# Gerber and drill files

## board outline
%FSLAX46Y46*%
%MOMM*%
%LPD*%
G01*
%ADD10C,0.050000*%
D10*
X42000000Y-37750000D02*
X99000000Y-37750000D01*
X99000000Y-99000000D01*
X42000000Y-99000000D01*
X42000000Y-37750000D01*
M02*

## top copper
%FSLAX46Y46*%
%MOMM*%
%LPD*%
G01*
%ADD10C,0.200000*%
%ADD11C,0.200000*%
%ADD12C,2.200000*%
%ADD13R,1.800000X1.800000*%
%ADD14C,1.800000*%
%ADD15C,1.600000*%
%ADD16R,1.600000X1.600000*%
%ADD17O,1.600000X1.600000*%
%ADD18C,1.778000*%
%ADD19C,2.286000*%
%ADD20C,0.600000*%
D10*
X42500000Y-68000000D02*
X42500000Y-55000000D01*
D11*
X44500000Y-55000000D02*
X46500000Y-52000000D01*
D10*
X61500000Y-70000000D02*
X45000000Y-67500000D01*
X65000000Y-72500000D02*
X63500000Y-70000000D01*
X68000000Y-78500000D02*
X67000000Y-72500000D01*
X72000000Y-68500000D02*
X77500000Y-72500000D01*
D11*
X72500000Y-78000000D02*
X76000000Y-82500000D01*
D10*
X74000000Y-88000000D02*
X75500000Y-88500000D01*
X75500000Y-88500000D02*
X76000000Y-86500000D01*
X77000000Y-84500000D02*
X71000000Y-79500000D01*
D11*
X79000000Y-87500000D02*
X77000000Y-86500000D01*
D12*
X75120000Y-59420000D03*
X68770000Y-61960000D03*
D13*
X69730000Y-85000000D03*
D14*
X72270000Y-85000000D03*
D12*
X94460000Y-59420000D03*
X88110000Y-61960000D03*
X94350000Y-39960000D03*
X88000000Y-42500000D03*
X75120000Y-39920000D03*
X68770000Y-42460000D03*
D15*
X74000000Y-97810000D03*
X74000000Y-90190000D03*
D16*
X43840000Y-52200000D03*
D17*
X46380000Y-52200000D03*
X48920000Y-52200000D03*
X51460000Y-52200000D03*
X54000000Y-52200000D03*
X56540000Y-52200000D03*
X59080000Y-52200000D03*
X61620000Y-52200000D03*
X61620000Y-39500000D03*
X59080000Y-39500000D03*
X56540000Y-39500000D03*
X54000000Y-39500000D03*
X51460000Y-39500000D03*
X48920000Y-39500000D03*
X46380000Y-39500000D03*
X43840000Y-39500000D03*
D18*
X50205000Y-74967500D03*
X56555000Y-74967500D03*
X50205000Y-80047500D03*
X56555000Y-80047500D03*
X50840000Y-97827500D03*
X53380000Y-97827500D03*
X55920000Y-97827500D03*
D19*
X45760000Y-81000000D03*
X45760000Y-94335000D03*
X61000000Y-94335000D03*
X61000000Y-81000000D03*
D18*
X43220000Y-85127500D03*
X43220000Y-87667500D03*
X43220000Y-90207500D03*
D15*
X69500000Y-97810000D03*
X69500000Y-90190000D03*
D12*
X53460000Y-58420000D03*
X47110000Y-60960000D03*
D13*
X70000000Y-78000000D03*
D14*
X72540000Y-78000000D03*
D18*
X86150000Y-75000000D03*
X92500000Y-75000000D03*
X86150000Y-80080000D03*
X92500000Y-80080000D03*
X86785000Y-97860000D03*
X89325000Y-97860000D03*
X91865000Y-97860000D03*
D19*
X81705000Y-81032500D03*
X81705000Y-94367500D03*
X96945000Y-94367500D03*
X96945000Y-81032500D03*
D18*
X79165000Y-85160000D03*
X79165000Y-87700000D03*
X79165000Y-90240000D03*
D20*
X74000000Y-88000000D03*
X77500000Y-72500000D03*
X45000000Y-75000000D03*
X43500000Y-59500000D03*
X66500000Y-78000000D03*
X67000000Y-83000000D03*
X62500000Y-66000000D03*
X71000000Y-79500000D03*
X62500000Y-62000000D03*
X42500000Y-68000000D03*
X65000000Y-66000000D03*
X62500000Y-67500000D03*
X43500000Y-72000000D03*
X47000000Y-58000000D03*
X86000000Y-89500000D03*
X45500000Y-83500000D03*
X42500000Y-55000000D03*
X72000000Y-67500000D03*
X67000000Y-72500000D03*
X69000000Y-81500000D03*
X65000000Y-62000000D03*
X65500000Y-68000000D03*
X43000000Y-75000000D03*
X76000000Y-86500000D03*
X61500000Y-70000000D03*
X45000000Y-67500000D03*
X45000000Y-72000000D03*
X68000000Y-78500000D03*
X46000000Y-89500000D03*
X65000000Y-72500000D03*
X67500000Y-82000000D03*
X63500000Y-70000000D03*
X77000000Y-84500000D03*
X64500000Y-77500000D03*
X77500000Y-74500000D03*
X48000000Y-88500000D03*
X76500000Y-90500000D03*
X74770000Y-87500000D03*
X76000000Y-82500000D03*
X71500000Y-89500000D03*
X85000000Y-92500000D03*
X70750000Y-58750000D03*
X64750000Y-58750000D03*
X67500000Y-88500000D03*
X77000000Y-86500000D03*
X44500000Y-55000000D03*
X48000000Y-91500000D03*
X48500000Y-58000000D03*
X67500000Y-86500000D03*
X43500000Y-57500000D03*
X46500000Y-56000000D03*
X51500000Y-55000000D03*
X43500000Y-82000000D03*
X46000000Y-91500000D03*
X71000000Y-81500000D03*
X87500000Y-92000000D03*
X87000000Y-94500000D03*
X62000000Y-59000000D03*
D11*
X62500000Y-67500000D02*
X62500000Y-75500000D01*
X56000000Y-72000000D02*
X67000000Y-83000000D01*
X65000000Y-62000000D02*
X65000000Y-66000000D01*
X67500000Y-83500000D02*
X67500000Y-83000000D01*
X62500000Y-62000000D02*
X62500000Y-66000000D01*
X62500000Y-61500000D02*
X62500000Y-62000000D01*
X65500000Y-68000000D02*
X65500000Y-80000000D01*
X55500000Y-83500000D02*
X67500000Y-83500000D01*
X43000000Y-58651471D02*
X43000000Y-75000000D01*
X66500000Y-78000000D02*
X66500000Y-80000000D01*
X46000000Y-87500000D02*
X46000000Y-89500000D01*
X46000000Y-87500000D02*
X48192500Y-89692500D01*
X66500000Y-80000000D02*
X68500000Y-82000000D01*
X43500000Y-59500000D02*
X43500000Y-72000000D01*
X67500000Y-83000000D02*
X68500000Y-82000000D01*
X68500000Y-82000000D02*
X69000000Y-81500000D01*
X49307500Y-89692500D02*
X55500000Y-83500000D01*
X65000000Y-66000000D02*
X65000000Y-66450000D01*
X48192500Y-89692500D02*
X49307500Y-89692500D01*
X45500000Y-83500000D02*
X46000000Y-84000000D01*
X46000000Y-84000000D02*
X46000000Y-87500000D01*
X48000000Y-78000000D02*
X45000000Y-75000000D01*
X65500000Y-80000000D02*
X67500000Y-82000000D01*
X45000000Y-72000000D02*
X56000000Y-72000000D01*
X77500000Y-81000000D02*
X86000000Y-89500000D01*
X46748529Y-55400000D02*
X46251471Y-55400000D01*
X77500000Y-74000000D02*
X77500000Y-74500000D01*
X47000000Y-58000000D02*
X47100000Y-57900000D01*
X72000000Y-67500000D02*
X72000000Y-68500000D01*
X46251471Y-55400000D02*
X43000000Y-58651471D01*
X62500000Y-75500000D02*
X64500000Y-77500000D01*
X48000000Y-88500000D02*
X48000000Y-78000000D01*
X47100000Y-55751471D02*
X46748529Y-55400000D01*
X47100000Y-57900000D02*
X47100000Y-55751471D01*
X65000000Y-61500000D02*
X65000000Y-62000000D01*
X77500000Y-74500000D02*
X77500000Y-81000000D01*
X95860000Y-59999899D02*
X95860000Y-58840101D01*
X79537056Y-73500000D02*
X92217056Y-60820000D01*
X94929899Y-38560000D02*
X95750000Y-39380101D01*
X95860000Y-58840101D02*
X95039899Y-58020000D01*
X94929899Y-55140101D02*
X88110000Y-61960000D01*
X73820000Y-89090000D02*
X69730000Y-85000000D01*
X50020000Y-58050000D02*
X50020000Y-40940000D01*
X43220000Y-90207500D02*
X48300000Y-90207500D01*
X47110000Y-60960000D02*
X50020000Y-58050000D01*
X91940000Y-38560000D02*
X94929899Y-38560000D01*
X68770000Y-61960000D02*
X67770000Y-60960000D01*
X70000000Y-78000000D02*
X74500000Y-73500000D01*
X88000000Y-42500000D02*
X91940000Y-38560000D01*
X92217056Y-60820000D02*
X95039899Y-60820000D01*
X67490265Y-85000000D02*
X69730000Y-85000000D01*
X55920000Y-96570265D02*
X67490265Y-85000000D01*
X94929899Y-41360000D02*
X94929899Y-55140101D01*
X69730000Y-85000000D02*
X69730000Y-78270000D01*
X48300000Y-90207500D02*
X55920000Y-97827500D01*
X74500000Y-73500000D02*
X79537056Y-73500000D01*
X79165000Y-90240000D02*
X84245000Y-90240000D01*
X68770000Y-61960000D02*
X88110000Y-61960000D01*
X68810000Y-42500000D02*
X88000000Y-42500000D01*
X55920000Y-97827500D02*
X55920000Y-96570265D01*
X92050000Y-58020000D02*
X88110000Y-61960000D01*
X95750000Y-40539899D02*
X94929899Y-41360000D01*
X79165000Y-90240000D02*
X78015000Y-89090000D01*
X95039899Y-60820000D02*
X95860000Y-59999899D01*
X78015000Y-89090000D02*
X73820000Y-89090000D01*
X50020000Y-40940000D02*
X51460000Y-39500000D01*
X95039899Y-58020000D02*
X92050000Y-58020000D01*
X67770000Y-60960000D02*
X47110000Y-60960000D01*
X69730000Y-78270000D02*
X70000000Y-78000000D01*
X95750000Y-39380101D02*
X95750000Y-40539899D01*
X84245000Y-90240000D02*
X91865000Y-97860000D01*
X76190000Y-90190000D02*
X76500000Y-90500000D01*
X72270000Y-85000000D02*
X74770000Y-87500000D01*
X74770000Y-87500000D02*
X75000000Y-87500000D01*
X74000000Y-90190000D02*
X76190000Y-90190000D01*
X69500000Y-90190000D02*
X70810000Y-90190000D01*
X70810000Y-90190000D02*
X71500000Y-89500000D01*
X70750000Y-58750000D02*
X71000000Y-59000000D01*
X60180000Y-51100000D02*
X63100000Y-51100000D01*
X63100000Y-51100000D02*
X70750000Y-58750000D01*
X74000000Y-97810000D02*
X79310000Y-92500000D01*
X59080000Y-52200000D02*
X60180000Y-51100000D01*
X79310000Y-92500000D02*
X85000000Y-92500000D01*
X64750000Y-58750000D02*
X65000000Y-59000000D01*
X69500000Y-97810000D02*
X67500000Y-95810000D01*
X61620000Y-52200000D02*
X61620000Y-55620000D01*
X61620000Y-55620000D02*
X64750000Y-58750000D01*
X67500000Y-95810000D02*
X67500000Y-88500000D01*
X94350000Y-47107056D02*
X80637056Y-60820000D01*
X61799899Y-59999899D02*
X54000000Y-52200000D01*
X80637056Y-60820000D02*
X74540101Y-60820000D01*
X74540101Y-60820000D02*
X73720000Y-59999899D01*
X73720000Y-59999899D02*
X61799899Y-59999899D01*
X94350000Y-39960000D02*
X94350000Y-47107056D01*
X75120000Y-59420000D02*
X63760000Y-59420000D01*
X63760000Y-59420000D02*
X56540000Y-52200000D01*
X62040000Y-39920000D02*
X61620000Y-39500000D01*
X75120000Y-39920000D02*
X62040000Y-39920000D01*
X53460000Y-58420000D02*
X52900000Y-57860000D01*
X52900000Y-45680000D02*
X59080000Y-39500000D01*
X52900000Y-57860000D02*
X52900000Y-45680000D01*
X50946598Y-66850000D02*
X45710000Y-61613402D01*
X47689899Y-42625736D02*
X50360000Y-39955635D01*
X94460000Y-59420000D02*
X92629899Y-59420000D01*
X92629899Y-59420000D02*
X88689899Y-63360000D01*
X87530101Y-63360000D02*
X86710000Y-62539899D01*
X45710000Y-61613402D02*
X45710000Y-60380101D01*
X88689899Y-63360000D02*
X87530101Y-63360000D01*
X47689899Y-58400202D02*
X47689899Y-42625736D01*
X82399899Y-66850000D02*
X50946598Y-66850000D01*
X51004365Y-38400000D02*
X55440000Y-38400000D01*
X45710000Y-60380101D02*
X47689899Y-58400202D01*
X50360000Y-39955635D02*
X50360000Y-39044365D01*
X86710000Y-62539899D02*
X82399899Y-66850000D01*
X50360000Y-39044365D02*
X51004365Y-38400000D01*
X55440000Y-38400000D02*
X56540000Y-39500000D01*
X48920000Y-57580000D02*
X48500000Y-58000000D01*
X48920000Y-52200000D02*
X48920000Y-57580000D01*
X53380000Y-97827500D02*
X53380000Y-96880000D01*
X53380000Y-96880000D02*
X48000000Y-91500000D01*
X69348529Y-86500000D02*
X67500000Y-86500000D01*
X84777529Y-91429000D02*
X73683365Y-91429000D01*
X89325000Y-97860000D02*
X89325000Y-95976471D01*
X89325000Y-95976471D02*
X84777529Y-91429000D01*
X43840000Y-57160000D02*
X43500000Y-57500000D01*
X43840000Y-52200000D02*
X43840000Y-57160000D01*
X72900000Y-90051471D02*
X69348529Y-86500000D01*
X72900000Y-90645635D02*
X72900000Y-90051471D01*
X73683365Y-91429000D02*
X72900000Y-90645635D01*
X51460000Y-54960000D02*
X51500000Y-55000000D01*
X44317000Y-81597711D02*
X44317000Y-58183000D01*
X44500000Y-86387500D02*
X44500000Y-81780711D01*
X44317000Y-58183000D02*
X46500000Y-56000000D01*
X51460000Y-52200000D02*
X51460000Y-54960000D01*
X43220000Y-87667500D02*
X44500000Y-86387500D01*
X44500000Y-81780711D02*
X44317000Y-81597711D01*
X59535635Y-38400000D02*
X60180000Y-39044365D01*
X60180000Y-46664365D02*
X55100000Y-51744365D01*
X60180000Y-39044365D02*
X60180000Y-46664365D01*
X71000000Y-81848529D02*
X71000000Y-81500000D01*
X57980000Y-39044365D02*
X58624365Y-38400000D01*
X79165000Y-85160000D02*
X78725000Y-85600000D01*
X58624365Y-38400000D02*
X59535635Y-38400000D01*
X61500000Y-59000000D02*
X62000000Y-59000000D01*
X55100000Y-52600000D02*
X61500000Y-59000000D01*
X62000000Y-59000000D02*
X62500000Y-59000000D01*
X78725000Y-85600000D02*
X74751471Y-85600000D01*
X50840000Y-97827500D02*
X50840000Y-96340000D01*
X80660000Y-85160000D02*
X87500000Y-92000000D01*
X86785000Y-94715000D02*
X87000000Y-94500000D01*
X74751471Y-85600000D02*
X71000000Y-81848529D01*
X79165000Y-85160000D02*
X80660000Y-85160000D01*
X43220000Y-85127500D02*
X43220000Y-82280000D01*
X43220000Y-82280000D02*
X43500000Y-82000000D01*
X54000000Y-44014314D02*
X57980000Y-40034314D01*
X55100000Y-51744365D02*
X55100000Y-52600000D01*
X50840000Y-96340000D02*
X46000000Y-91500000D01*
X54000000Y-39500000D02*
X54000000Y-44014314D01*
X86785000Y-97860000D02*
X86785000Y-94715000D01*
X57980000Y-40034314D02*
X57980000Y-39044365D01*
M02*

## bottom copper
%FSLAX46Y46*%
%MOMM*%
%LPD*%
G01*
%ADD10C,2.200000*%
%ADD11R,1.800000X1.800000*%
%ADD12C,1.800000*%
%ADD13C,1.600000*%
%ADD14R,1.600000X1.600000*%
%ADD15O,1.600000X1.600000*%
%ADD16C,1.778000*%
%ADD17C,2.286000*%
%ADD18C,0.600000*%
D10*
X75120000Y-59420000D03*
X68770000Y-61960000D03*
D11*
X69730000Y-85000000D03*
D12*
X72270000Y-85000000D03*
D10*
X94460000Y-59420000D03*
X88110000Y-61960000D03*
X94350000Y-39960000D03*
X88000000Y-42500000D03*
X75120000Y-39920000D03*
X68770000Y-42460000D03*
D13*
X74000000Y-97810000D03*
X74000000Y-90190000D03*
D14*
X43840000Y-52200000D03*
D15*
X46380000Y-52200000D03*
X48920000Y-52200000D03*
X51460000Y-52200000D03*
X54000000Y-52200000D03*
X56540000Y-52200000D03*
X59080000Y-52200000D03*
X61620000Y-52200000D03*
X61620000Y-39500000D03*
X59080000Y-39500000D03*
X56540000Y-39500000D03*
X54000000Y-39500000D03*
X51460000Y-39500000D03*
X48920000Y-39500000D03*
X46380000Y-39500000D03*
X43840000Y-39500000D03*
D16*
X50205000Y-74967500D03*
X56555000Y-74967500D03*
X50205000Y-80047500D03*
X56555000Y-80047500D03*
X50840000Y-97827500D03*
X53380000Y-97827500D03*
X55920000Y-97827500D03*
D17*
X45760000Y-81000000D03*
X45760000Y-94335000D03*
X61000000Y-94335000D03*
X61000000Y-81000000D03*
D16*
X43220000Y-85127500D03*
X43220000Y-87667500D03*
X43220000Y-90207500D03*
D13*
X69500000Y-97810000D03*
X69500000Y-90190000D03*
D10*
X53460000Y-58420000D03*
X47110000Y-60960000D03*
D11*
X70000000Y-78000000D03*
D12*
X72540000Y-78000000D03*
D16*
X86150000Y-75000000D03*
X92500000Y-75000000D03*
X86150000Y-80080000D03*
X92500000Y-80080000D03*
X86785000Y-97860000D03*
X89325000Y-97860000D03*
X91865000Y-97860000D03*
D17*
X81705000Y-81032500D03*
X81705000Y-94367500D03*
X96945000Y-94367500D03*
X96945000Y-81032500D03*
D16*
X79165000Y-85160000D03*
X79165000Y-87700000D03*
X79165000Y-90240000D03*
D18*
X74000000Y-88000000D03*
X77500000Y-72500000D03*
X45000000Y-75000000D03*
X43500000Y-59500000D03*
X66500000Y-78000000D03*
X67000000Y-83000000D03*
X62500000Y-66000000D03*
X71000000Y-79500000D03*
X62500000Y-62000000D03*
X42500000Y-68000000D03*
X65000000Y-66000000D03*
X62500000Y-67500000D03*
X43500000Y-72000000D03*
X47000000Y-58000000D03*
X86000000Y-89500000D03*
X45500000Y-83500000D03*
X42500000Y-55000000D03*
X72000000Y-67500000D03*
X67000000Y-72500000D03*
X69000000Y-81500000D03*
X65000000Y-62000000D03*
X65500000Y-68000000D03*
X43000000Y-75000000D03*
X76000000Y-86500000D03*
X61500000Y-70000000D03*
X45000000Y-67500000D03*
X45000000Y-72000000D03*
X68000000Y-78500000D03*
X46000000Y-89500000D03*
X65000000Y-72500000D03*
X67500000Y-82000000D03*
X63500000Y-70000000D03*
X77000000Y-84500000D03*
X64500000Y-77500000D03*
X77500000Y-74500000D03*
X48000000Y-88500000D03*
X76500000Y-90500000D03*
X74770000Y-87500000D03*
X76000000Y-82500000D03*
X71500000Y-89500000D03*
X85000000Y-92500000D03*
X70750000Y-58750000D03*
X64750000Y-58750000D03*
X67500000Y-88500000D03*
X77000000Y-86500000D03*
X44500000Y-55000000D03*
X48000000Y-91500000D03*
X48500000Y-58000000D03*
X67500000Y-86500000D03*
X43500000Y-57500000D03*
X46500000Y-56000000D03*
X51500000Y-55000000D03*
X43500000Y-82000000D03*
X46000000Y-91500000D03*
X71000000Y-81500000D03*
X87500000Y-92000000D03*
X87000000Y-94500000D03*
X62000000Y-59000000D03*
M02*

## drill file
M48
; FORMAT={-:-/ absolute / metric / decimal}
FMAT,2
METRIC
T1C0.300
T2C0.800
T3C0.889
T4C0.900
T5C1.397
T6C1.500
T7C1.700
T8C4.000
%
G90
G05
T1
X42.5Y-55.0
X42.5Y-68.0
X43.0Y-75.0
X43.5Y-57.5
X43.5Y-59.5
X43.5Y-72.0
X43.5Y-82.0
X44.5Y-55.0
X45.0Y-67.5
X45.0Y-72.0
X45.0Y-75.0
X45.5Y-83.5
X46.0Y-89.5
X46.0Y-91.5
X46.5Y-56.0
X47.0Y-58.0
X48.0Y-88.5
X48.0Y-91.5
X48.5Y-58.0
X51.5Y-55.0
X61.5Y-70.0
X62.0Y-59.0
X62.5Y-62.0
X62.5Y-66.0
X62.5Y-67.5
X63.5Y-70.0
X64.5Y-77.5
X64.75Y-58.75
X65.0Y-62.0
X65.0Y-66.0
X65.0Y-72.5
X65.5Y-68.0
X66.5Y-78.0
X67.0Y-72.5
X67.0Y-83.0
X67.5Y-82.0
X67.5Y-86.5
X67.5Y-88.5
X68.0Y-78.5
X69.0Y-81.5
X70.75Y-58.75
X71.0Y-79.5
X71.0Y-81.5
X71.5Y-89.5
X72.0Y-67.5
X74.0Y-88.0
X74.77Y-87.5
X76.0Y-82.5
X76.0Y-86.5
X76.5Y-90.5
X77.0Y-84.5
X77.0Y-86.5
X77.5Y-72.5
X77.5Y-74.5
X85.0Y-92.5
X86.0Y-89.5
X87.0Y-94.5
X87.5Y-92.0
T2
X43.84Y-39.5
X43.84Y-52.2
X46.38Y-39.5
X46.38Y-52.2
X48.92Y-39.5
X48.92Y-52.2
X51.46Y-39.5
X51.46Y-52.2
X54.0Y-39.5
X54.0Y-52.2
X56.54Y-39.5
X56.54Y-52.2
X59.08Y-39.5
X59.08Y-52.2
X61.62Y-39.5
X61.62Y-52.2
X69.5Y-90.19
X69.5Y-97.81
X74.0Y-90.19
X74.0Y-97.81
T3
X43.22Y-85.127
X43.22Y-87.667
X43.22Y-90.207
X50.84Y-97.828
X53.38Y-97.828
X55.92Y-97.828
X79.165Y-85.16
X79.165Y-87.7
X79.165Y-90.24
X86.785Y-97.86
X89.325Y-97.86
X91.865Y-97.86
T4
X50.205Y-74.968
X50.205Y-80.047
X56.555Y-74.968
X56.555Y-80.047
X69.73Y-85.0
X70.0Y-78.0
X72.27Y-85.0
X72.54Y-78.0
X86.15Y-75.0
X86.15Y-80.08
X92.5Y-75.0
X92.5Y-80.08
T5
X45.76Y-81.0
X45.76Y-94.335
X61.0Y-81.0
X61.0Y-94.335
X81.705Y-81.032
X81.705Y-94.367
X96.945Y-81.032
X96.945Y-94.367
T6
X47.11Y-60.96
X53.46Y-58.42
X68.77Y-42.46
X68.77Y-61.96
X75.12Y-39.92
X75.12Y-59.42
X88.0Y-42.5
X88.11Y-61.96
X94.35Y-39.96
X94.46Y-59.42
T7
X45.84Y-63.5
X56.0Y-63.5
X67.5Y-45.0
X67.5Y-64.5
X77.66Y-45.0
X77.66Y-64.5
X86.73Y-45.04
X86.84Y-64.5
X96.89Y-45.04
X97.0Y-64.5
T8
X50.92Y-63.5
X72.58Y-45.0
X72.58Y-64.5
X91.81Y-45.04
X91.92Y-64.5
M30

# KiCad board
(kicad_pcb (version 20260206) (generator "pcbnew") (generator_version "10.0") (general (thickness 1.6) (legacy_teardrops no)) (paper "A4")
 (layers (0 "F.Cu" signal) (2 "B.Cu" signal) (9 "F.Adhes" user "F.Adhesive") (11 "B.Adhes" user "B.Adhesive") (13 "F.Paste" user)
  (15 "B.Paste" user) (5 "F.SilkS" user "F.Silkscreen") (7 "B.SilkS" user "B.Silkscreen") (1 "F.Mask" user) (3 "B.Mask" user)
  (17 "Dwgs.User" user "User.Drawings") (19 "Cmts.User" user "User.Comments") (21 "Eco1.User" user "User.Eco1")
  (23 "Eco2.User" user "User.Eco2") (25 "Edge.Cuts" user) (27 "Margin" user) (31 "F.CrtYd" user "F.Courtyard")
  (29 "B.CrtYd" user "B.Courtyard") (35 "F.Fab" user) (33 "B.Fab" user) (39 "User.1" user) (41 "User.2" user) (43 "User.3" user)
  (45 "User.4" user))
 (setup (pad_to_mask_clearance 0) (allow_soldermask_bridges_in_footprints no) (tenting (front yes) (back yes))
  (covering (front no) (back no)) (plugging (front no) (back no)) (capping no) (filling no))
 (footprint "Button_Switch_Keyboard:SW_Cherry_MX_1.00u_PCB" (layer "F.Cu") (at 75.12 59.42)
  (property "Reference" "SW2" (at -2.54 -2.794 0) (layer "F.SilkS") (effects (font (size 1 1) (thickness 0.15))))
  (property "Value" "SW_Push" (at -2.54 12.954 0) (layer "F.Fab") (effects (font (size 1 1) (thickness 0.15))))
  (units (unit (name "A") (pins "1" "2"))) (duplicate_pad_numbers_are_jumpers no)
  (pad "" np_thru_hole circle (at -7.62 5.08) (size 1.7 1.7) (drill 1.7) (layers "*.Cu" "*.Mask"))
  (pad "" np_thru_hole circle (at -2.54 5.08) (size 4 4) (drill 4) (layers "*.Cu" "*.Mask"))
  (pad "" np_thru_hole circle (at 2.54 5.08) (size 1.7 1.7) (drill 1.7) (layers "*.Cu" "*.Mask"))
  (pad "1" thru_hole circle (at 0 0) (size 2.2 2.2) (drill 1.5) (layers "*.Cu" "*.Mask") (remove_unused_layers no) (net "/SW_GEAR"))
  (pad "2" thru_hole circle (at -6.35 2.54) (size 2.2 2.2) (drill 1.5) (layers "*.Cu" "*.Mask") (remove_unused_layers no) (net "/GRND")))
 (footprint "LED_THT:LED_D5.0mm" (layer "F.Cu") (at 69.73 85)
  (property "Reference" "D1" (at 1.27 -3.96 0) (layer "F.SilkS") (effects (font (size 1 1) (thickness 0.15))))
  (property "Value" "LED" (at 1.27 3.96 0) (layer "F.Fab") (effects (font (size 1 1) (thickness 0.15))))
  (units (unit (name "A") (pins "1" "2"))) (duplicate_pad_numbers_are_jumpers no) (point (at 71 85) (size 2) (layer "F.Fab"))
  (pad "1" thru_hole rect (at 0 0) (size 1.8 1.8) (drill 0.9) (layers "*.Cu" "*.Mask") (remove_unused_layers no) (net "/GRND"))
  (pad "2" thru_hole circle (at 2.54 0) (size 1.8 1.8) (drill 0.9) (layers "*.Cu" "*.Mask") (remove_unused_layers no) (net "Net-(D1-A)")))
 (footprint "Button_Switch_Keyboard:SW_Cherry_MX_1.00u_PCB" (layer "F.Cu") (at 94.46 59.42)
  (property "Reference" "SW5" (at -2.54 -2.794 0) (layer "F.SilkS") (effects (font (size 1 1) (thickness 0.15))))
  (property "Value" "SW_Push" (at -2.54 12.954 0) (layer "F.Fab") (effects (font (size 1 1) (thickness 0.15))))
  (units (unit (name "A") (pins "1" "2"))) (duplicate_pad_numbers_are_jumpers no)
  (pad "" np_thru_hole circle (at -7.62 5.08) (size 1.7 1.7) (drill 1.7) (layers "*.Cu" "*.Mask"))
  (pad "" np_thru_hole circle (at -2.54 5.08) (size 4 4) (drill 4) (layers "*.Cu" "*.Mask"))
  (pad "" np_thru_hole circle (at 2.54 5.08) (size 1.7 1.7) (drill 1.7) (layers "*.Cu" "*.Mask"))
  (pad "1" thru_hole circle (at 0 0) (size 2.2 2.2) (drill 1.5) (layers "*.Cu" "*.Mask") (remove_unused_layers no) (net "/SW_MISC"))
  (pad "2" thru_hole circle (at -6.35 2.54) (size 2.2 2.2) (drill 1.5) (layers "*.Cu" "*.Mask") (remove_unused_layers no) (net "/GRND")))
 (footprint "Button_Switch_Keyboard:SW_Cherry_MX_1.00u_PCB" (layer "F.Cu") (at 94.35 39.96)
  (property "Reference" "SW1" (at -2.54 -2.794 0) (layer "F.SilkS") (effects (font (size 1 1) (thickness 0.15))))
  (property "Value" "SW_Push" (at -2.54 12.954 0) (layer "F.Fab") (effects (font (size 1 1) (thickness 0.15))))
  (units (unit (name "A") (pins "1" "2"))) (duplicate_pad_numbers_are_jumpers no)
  (pad "" np_thru_hole circle (at -7.62 5.08) (size 1.7 1.7) (drill 1.7) (layers "*.Cu" "*.Mask"))
  (pad "" np_thru_hole circle (at -2.54 5.08) (size 4 4) (drill 4) (layers "*.Cu" "*.Mask"))
  (pad "" np_thru_hole circle (at 2.54 5.08) (size 1.7 1.7) (drill 1.7) (layers "*.Cu" "*.Mask"))
  (pad "1" thru_hole circle (at 0 0) (size 2.2 2.2) (drill 1.5) (layers "*.Cu" "*.Mask") (remove_unused_layers no) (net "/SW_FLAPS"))
  (pad "2" thru_hole circle (at -6.35 2.54) (size 2.2 2.2) (drill 1.5) (layers "*.Cu" "*.Mask") (remove_unused_layers no) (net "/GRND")))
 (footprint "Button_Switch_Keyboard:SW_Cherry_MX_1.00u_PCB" (layer "F.Cu") (at 75.12 39.92)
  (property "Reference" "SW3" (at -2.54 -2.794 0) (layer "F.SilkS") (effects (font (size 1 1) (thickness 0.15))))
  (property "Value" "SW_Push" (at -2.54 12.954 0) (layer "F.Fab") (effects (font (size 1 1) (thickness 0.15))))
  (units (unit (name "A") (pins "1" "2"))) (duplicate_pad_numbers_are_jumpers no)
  (pad "" np_thru_hole circle (at -7.62 5.08) (size 1.7 1.7) (drill 1.7) (layers "*.Cu" "*.Mask"))
  (pad "" np_thru_hole circle (at -2.54 5.08) (size 4 4) (drill 4) (layers "*.Cu" "*.Mask"))
  (pad "" np_thru_hole circle (at 2.54 5.08) (size 1.7 1.7) (drill 1.7) (layers "*.Cu" "*.Mask"))
  (pad "1" thru_hole circle (at 0 0) (size 2.2 2.2) (drill 1.5) (layers "*.Cu" "*.Mask") (remove_unused_layers no) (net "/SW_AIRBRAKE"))
  (pad "2" thru_hole circle (at -6.35 2.54) (size 2.2 2.2) (drill 1.5) (layers "*.Cu" "*.Mask") (remove_unused_layers no) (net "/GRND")))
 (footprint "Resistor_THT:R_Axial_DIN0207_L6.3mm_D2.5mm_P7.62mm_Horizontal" (layer "F.Cu") (at 74 97.81 90)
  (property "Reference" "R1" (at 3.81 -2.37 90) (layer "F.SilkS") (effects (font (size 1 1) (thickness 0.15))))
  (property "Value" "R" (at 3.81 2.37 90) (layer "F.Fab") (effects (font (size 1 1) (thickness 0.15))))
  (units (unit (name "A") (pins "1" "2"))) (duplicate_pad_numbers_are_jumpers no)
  (pad "1" thru_hole circle (at 0 0 90) (size 1.6 1.6) (drill 0.8) (layers "*.Cu" "*.Mask") (remove_unused_layers no) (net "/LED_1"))
  (pad "2" thru_hole circle (at 7.62 0 90) (size 1.6 1.6) (drill 0.8) (layers "*.Cu" "*.Mask") (remove_unused_layers no) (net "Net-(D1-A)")))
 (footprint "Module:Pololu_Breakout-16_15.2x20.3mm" (layer "F.Cu") (at 43.84 52.2 90)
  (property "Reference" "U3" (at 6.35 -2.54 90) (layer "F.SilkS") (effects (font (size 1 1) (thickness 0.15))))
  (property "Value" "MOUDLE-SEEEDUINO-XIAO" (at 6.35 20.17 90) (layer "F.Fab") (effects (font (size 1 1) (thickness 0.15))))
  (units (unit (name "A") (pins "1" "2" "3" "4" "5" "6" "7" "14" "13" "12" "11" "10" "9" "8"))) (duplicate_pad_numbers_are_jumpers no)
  (pad "1" thru_hole rect (at 0 0 90) (size 1.6 1.6) (drill 0.8) (layers "*.Cu" "*.Mask") (remove_unused_layers no) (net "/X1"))
  (pad "2" thru_hole oval (at 0 2.54 90) (size 1.6 1.6) (drill 0.8) (layers "*.Cu" "*.Mask") (remove_unused_layers no) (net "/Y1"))
  (pad "3" thru_hole oval (at 0 5.08 90) (size 1.6 1.6) (drill 0.8) (layers "*.Cu" "*.Mask") (remove_unused_layers no) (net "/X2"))
  (pad "4" thru_hole oval (at 0 7.62 90) (size 1.6 1.6) (drill 0.8) (layers "*.Cu" "*.Mask") (remove_unused_layers no) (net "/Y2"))
  (pad "5" thru_hole oval (at 0 10.16 90) (size 1.6 1.6) (drill 0.8) (layers "*.Cu" "*.Mask") (remove_unused_layers no) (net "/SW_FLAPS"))
  (pad "6" thru_hole oval (at 0 12.7 90) (size 1.6 1.6) (drill 0.8) (layers "*.Cu" "*.Mask") (remove_unused_layers no) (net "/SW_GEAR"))
  (pad "7" thru_hole oval (at 0 15.24 90) (size 1.6 1.6) (drill 0.8) (layers "*.Cu" "*.Mask") (remove_unused_layers no) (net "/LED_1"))
  (pad "8" thru_hole oval (at 0 17.78 90) (size 1.6 1.6) (drill 0.8) (layers "*.Cu" "*.Mask") (remove_unused_layers no) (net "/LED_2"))
  (pad "9" thru_hole oval (at 12.7 17.78 90) (size 1.6 1.6) (drill 0.8) (layers "*.Cu" "*.Mask") (remove_unused_layers no)
   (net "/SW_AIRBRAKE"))
  (pad "10" thru_hole oval (at 12.7 15.24 90) (size 1.6 1.6) (drill 0.8) (layers "*.Cu" "*.Mask") (remove_unused_layers no)
   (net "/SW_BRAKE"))
  (pad "11" thru_hole oval (at 12.7 12.7 90) (size 1.6 1.6) (drill 0.8) (layers "*.Cu" "*.Mask") (remove_unused_layers no) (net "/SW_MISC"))
  (pad "12" thru_hole oval (at 12.7 10.16 90) (size 1.6 1.6) (drill 0.8) (layers "*.Cu" "*.Mask") (remove_unused_layers no) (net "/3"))
  (pad "13" thru_hole oval (at 12.7 7.62 90) (size 1.6 1.6) (drill 0.8) (layers "*.Cu" "*.Mask") (remove_unused_layers no) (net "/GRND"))
  (pad "14" thru_hole oval (at 12.7 5.08 90) (size 1.6 1.6) (drill 0.8) (layers "*.Cu" "*.Mask") (remove_unused_layers no)
   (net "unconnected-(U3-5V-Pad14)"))
  (pad "15" thru_hole oval (at 12.7 2.54 90) (size 1.6 1.6) (drill 0.8) (layers "*.Cu" "*.Mask") (remove_unused_layers no))
  (pad "16" thru_hole oval (at 12.7 0 90) (size 1.6 1.6) (drill 0.8) (layers "*.Cu" "*.Mask") (remove_unused_layers no)))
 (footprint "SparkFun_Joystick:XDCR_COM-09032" (layer "F.Cu") (at 53.38 87.6675)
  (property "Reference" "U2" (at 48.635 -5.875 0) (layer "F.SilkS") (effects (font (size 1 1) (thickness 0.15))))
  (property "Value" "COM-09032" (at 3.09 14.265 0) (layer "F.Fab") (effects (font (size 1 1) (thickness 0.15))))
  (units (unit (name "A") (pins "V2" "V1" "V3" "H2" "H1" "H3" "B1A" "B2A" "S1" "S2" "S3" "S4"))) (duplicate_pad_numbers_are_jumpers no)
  (pad "B1A" thru_hole circle (at -3.175 -12.7) (size 1.778 1.778) (drill 0.9) (layers "*.Cu" "*.Mask") (remove_unused_layers no)
   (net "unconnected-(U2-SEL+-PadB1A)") (solder_mask_margin 0.102))
  (pad "B1B" thru_hole circle (at 3.175 -12.7) (size 1.778 1.778) (drill 0.9) (layers "*.Cu" "*.Mask") (remove_unused_layers no)
   (solder_mask_margin 0.102))
  (pad "B2A" thru_hole circle (at -3.175 -7.62) (size 1.778 1.778) (drill 0.9) (layers "*.Cu" "*.Mask") (remove_unused_layers no)
   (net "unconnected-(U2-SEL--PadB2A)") (solder_mask_margin 0.102))
  (pad "B2B" thru_hole circle (at 3.175 -7.62) (size 1.778 1.778) (drill 0.9) (layers "*.Cu" "*.Mask") (remove_unused_layers no)
   (solder_mask_margin 0.102))
  (pad "H1" thru_hole circle (at -2.54 10.16) (size 1.778 1.778) (drill 0.889) (layers "*.Cu" "*.Mask") (remove_unused_layers no) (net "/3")
   (solder_mask_margin 0.102))
  (pad "H2" thru_hole circle (at 0 10.16) (size 1.778 1.778) (drill 0.889) (layers "*.Cu" "*.Mask") (remove_unused_layers no) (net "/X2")
   (solder_mask_margin 0.102))
  (pad "H3" thru_hole circle (at 2.54 10.16) (size 1.778 1.778) (drill 0.889) (layers "*.Cu" "*.Mask") (remove_unused_layers no)
   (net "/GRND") (solder_mask_margin 0.102))
  (pad "S1" thru_hole circle (at -7.62 -6.6675) (size 2.286 2.286) (drill 1.397) (layers "*.Cu" "*.Mask") (remove_unused_layers no)
   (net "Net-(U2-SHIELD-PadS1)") (solder_mask_margin 0.102))
  (pad "S2" thru_hole circle (at -7.62 6.6675) (size 2.286 2.286) (drill 1.397) (layers "*.Cu" "*.Mask") (remove_unused_layers no)
   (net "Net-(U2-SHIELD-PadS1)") (solder_mask_margin 0.102))
  (pad "S3" thru_hole circle (at 7.62 6.6675) (size 2.286 2.286) (drill 1.397) (layers "*.Cu" "*.Mask") (remove_unused_layers no)
   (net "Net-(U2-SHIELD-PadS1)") (solder_mask_margin 0.102))
  (pad "S4" thru_hole circle (at 7.62 -6.6675) (size 2.286 2.286) (drill 1.397) (layers "*.Cu" "*.Mask") (remove_unused_layers no)
   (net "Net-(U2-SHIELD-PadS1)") (solder_mask_margin 0.102))
  (pad "V1" thru_hole circle (at -10.16 -2.54) (size 1.778 1.778) (drill 0.889) (layers "*.Cu" "*.Mask") (remove_unused_layers no)
   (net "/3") (solder_mask_margin 0.102))
  (pad "V2" thru_hole circle (at -10.16 0) (size 1.778 1.778) (drill 0.889) (layers "*.Cu" "*.Mask") (remove_unused_layers no) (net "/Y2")
   (solder_mask_margin 0.102))
  (pad "V3" thru_hole circle (at -10.16 2.54) (size 1.778 1.778) (drill 0.889) (layers "*.Cu" "*.Mask") (remove_unused_layers no)
   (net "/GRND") (solder_mask_margin 0.102)))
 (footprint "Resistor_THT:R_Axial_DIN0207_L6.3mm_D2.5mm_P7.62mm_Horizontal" (layer "F.Cu") (at 69.5 97.81 90)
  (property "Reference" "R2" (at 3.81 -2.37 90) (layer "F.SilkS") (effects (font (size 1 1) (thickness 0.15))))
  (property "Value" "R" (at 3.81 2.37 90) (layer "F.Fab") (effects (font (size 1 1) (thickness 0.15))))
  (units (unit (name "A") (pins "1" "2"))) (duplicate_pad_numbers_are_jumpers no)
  (pad "1" thru_hole circle (at 0 0 90) (size 1.6 1.6) (drill 0.8) (layers "*.Cu" "*.Mask") (remove_unused_layers no) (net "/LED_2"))
  (pad "2" thru_hole circle (at 7.62 0 90) (size 1.6 1.6) (drill 0.8) (layers "*.Cu" "*.Mask") (remove_unused_layers no) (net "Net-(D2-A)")))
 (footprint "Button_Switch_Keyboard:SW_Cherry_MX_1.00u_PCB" (layer "F.Cu") (at 53.46 58.42)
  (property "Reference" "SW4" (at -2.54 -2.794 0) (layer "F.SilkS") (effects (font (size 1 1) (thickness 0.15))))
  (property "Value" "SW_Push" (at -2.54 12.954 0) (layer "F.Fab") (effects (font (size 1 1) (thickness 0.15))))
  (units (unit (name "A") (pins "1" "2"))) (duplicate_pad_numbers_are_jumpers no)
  (pad "" np_thru_hole circle (at -7.62 5.08) (size 1.7 1.7) (drill 1.7) (layers "*.Cu" "*.Mask"))
  (pad "" np_thru_hole circle (at -2.54 5.08) (size 4 4) (drill 4) (layers "*.Cu" "*.Mask"))
  (pad "" np_thru_hole circle (at 2.54 5.08) (size 1.7 1.7) (drill 1.7) (layers "*.Cu" "*.Mask"))
  (pad "1" thru_hole circle (at 0 0) (size 2.2 2.2) (drill 1.5) (layers "*.Cu" "*.Mask") (remove_unused_layers no) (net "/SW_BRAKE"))
  (pad "2" thru_hole circle (at -6.35 2.54) (size 2.2 2.2) (drill 1.5) (layers "*.Cu" "*.Mask") (remove_unused_layers no) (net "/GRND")))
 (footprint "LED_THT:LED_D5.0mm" (layer "F.Cu") (at 70 78)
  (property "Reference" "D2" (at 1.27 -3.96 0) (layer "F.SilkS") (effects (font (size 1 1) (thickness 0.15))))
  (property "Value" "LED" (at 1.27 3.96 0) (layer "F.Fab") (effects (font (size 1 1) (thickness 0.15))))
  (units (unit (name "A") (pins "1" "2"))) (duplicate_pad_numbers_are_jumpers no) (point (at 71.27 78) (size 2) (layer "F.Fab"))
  (pad "1" thru_hole rect (at 0 0) (size 1.8 1.8) (drill 0.9) (layers "*.Cu" "*.Mask") (remove_unused_layers no) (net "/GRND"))
  (pad "2" thru_hole circle (at 2.54 0) (size 1.8 1.8) (drill 0.9) (layers "*.Cu" "*.Mask") (remove_unused_layers no) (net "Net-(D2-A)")))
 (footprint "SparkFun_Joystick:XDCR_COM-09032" (layer "F.Cu") (at 89.325 87.7)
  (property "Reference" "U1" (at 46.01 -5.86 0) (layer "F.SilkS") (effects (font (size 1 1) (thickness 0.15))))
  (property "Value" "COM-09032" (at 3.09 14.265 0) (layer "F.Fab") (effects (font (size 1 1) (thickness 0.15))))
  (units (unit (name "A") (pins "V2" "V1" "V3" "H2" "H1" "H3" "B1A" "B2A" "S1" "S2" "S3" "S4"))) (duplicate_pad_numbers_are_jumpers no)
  (pad "B1A" thru_hole circle (at -3.175 -12.7) (size 1.778 1.778) (drill 0.9) (layers "*.Cu" "*.Mask") (remove_unused_layers no)
   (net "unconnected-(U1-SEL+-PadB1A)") (solder_mask_margin 0.102))
  (pad "B1B" thru_hole circle (at 3.175 -12.7) (size 1.778 1.778) (drill 0.9) (layers "*.Cu" "*.Mask") (remove_unused_layers no)
   (solder_mask_margin 0.102))
  (pad "B2A" thru_hole circle (at -3.175 -7.62) (size 1.778 1.778) (drill 0.9) (layers "*.Cu" "*.Mask") (remove_unused_layers no)
   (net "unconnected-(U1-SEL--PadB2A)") (solder_mask_margin 0.102))
  (pad "B2B" thru_hole circle (at 3.175 -7.62) (size 1.778 1.778) (drill 0.9) (layers "*.Cu" "*.Mask") (remove_unused_layers no)
   (solder_mask_margin 0.102))
  (pad "H1" thru_hole circle (at -2.54 10.16) (size 1.778 1.778) (drill 0.889) (layers "*.Cu" "*.Mask") (remove_unused_layers no) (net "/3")
   (solder_mask_margin 0.102))
  (pad "H2" thru_hole circle (at 0 10.16) (size 1.778 1.778) (drill 0.889) (layers "*.Cu" "*.Mask") (remove_unused_layers no) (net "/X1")
   (solder_mask_margin 0.102))
  (pad "H3" thru_hole circle (at 2.54 10.16) (size 1.778 1.778) (drill 0.889) (layers "*.Cu" "*.Mask") (remove_unused_layers no)
   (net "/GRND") (solder_mask_margin 0.102))
  (pad "S1" thru_hole circle (at -7.62 -6.6675) (size 2.286 2.286) (drill 1.397) (layers "*.Cu" "*.Mask") (remove_unused_layers no)
   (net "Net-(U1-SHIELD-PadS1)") (solder_mask_margin 0.102))
  (pad "S2" thru_hole circle (at -7.62 6.6675) (size 2.286 2.286) (drill 1.397) (layers "*.Cu" "*.Mask") (remove_unused_layers no)
   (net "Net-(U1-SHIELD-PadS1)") (solder_mask_margin 0.102))
  (pad "S3" thru_hole circle (at 7.62 6.6675) (size 2.286 2.286) (drill 1.397) (layers "*.Cu" "*.Mask") (remove_unused_layers no)
   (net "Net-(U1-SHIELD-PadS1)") (solder_mask_margin 0.102))
  (pad "S4" thru_hole circle (at 7.62 -6.6675) (size 2.286 2.286) (drill 1.397) (layers "*.Cu" "*.Mask") (remove_unused_layers no)
   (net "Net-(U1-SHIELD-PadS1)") (solder_mask_margin 0.102))
  (pad "V1" thru_hole circle (at -10.16 -2.54) (size 1.778 1.778) (drill 0.889) (layers "*.Cu" "*.Mask") (remove_unused_layers no)
   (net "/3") (solder_mask_margin 0.102))
  (pad "V2" thru_hole circle (at -10.16 0) (size 1.778 1.778) (drill 0.889) (layers "*.Cu" "*.Mask") (remove_unused_layers no) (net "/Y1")
   (solder_mask_margin 0.102))
  (pad "V3" thru_hole circle (at -10.16 2.54) (size 1.778 1.778) (drill 0.889) (layers "*.Cu" "*.Mask") (remove_unused_layers no)
   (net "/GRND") (solder_mask_margin 0.102)))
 (gr_line (start 42.5 68) (end 42.5 55) (stroke (width 0.2) (type default)) (layer "F.Cu"))
 (gr_line (start 44.5 55) (end 46.5 52) (stroke (width 0.2) (type default)) (layer "F.Cu") (net "/Y1"))
 (gr_line (start 61.5 70) (end 45 67.5) (stroke (width 0.2) (type default)) (layer "F.Cu"))
 (gr_line (start 65 72.5) (end 63.5 70) (stroke (width 0.2) (type default)) (layer "F.Cu"))
 (gr_line (start 68 78.5) (end 67 72.5) (stroke (width 0.2) (type default)) (layer "F.Cu"))
 (gr_line (start 72 68.5) (end 77.5 72.5) (stroke (width 0.2) (type default)) (layer "F.Cu"))
 (gr_line (start 72.5 78) (end 76 82.5) (stroke (width 0.2) (type default)) (layer "F.Cu") (net "Net-(D2-A)"))
 (gr_line (start 74 88) (end 75.5 88.5) (stroke (width 0.2) (type default)) (layer "F.Cu"))
 (gr_line (start 75.5 88.5) (end 76 86.5) (stroke (width 0.2) (type default)) (layer "F.Cu"))
 (gr_line (start 77 84.5) (end 71 79.5) (stroke (width 0.2) (type default)) (layer "F.Cu"))
 (gr_line (start 79 87.5) (end 77 86.5) (stroke (width 0.2) (type default)) (layer "F.Cu") (net "/Y1"))
 (gr_rect (start 42 37.75) (end 99 99) (stroke (width 0.05) (type solid)) (fill no) (layer "Edge.Cuts"))
 (segment (start 62.5 67.5) (end 62.5 75.5) (width 0.2) (layer "F.Cu") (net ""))
 (segment (start 56 72) (end 67 83) (width 0.2) (layer "F.Cu") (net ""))
 (segment (start 65 62) (end 65 66) (width 0.2) (layer "F.Cu") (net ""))
 (segment (start 67.5 83.5) (end 67.5 83) (width 0.2) (layer "F.Cu") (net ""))
 (segment (start 62.5 62) (end 62.5 66) (width 0.2) (layer "F.Cu") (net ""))
 (segment (start 62.5 61.5) (end 62.5 62) (width 0.2) (layer "F.Cu") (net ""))
 (segment (start 65.5 68) (end 65.5 80) (width 0.2) (layer "F.Cu") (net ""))
 (segment (start 55.5 83.5) (end 67.5 83.5) (width 0.2) (layer "F.Cu") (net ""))
 (segment (start 43 58.651471) (end 43 75) (width 0.2) (layer "F.Cu") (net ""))
 (segment (start 66.5 78) (end 66.5 80) (width 0.2) (layer "F.Cu") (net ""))
 (segment (start 46 87.5) (end 46 89.5) (width 0.2) (layer "F.Cu") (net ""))
 (segment (start 46 87.5) (end 48.1925 89.6925) (width 0.2) (layer "F.Cu") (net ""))
 (segment (start 66.5 80) (end 68.5 82) (width 0.2) (layer "F.Cu") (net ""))
 (segment (start 43.5 59.5) (end 43.5 72) (width 0.2) (layer "F.Cu") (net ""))
 (segment (start 67.5 83) (end 68.5 82) (width 0.2) (layer "F.Cu") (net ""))
 (segment (start 68.5 82) (end 69 81.5) (width 0.2) (layer "F.Cu") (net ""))
 (segment (start 49.3075 89.6925) (end 55.5 83.5) (width 0.2) (layer "F.Cu") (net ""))
 (segment (start 65 66) (end 65 66.45) (width 0.2) (layer "F.Cu") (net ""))
 (segment (start 48.1925 89.6925) (end 49.3075 89.6925) (width 0.2) (layer "F.Cu") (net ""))
 (segment (start 45.5 83.5) (end 46 84) (width 0.2) (layer "F.Cu") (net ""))
 (segment (start 46 84) (end 46 87.5) (width 0.2) (layer "F.Cu") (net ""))
 (segment (start 48 78) (end 45 75) (width 0.2) (layer "F.Cu") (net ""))
 (segment (start 65.5 80) (end 67.5 82) (width 0.2) (layer "F.Cu") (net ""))
 (segment (start 45 72) (end 56 72) (width 0.2) (layer "F.Cu") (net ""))
 (segment (start 77.5 81) (end 86 89.5) (width 0.2) (layer "F.Cu") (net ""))
 (segment (start 46.748529 55.4) (end 46.251471 55.4) (width 0.2) (layer "F.Cu") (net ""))
 (segment (start 77.5 74) (end 77.5 74.5) (width 0.2) (layer "F.Cu") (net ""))
 (segment (start 47 58) (end 47.1 57.9) (width 0.2) (layer "F.Cu") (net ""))
 (segment (start 72 67.5) (end 72 68.5) (width 0.2) (layer "F.Cu") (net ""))
 (segment (start 46.251471 55.4) (end 43 58.651471) (width 0.2) (layer "F.Cu") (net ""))
 (segment (start 62.5 75.5) (end 64.5 77.5) (width 0.2) (layer "F.Cu") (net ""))
 (segment (start 48 88.5) (end 48 78) (width 0.2) (layer "F.Cu") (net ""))
 (segment (start 47.1 55.751471) (end 46.748529 55.4) (width 0.2) (layer "F.Cu") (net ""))
 (segment (start 47.1 57.9) (end 47.1 55.751471) (width 0.2) (layer "F.Cu") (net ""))
 (segment (start 65 61.5) (end 65 62) (width 0.2) (layer "F.Cu") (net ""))
 (segment (start 77.5 74.5) (end 77.5 81) (width 0.2) (layer "F.Cu") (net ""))
 (via (at 74 88) (size 0.6) (drill 0.3) (layers "F.Cu" "B.Cu") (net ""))
 (via (at 77.5 72.5) (size 0.6) (drill 0.3) (layers "F.Cu" "B.Cu") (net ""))
 (via (at 45 75) (size 0.6) (drill 0.3) (layers "F.Cu" "B.Cu") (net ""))
 (via (at 43.5 59.5) (size 0.6) (drill 0.3) (layers "F.Cu" "B.Cu") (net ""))
 (via (at 66.5 78) (size 0.6) (drill 0.3) (layers "F.Cu" "B.Cu") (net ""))
 (via (at 67 83) (size 0.6) (drill 0.3) (layers "F.Cu" "B.Cu") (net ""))
 (via (at 62.5 66) (size 0.6) (drill 0.3) (layers "F.Cu" "B.Cu") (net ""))
 (via (at 71 79.5) (size 0.6) (drill 0.3) (layers "F.Cu" "B.Cu") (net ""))
 (via (at 62.5 62) (size 0.6) (drill 0.3) (layers "F.Cu" "B.Cu") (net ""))
 (via (at 42.5 68) (size 0.6) (drill 0.3) (layers "F.Cu" "B.Cu") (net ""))
 (via (at 65 66) (size 0.6) (drill 0.3) (layers "F.Cu" "B.Cu") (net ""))
 (via (at 62.5 67.5) (size 0.6) (drill 0.3) (layers "F.Cu" "B.Cu") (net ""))
 (via (at 43.5 72) (size 0.6) (drill 0.3) (layers "F.Cu" "B.Cu") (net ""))
 (via (at 47 58) (size 0.6) (drill 0.3) (layers "F.Cu" "B.Cu") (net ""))
 (via (at 86 89.5) (size 0.6) (drill 0.3) (layers "F.Cu" "B.Cu") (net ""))
 (via (at 45.5 83.5) (size 0.6) (drill 0.3) (layers "F.Cu" "B.Cu") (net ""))
 (via (at 42.5 55) (size 0.6) (drill 0.3) (layers "F.Cu" "B.Cu") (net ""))
 (via (at 72 67.5) (size 0.6) (drill 0.3) (layers "F.Cu" "B.Cu") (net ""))
 (via (at 67 72.5) (size 0.6) (drill 0.3) (layers "F.Cu" "B.Cu") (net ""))
 (via (at 69 81.5) (size 0.6) (drill 0.3) (layers "F.Cu" "B.Cu") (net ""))
 (via (at 65 62) (size 0.6) (drill 0.3) (layers "F.Cu" "B.Cu") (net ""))
 (via (at 65.5 68) (size 0.6) (drill 0.3) (layers "F.Cu" "B.Cu") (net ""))
 (via (at 43 75) (size 0.6) (drill 0.3) (layers "F.Cu" "B.Cu") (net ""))
 (via (at 76 86.5) (size 0.6) (drill 0.3) (layers "F.Cu" "B.Cu") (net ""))
 (via (at 61.5 70) (size 0.6) (drill 0.3) (layers "F.Cu" "B.Cu") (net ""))
 (via (at 45 67.5) (size 0.6) (drill 0.3) (layers "F.Cu" "B.Cu") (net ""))
 (via (at 45 72) (size 0.6) (drill 0.3) (layers "F.Cu" "B.Cu") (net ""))
 (via (at 68 78.5) (size 0.6) (drill 0.3) (layers "F.Cu" "B.Cu") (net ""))
 (via (at 46 89.5) (size 0.6) (drill 0.3) (layers "F.Cu" "B.Cu") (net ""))
 (via (at 65 72.5) (size 0.6) (drill 0.3) (layers "F.Cu" "B.Cu") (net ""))
 (via (at 67.5 82) (size 0.6) (drill 0.3) (layers "F.Cu" "B.Cu") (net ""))
 (via (at 63.5 70) (size 0.6) (drill 0.3) (layers "F.Cu" "B.Cu") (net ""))
 (via (at 77 84.5) (size 0.6) (drill 0.3) (layers "F.Cu" "B.Cu") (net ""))
 (via (at 64.5 77.5) (size 0.6) (drill 0.3) (layers "F.Cu" "B.Cu") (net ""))
 (via (at 77.5 74.5) (size 0.6) (drill 0.3) (layers "F.Cu" "B.Cu") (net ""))
 (via (at 48 88.5) (size 0.6) (drill 0.3) (layers "F.Cu" "B.Cu") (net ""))
 (segment (start 95.86 59.999899) (end 95.86 58.840101) (width 0.2) (layer "F.Cu") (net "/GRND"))
 (segment (start 79.537056 73.5) (end 92.217056 60.82) (width 0.2) (layer "F.Cu") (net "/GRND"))
 (segment (start 94.929899 38.56) (end 95.75 39.380101) (width 0.2) (layer "F.Cu") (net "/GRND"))
 (segment (start 95.86 58.840101) (end 95.039899 58.02) (width 0.2) (layer "F.Cu") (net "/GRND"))
 (segment (start 94.929899 55.140101) (end 88.11 61.96) (width 0.2) (layer "F.Cu") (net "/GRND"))
 (segment (start 73.82 89.09) (end 69.73 85) (width 0.2) (layer "F.Cu") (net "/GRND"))
 (segment (start 50.02 58.05) (end 50.02 40.94) (width 0.2) (layer "F.Cu") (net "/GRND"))
 (segment (start 43.22 90.2075) (end 48.3 90.2075) (width 0.2) (layer "F.Cu") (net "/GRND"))
 (segment (start 47.11 60.96) (end 50.02 58.05) (width 0.2) (layer "F.Cu") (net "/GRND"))
 (segment (start 91.94 38.56) (end 94.929899 38.56) (width 0.2) (layer "F.Cu") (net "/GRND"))
 (segment (start 68.77 61.96) (end 67.77 60.96) (width 0.2) (layer "F.Cu") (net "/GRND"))
 (segment (start 70 78) (end 74.5 73.5) (width 0.2) (layer "F.Cu") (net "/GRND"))
 (segment (start 88 42.5) (end 91.94 38.56) (width 0.2) (layer "F.Cu") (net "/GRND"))
 (segment (start 92.217056 60.82) (end 95.039899 60.82) (width 0.2) (layer "F.Cu") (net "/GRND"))
 (segment (start 67.490265 85) (end 69.73 85) (width 0.2) (layer "F.Cu") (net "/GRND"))
 (segment (start 55.92 96.570265) (end 67.490265 85) (width 0.2) (layer "F.Cu") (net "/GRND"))
 (segment (start 94.929899 41.36) (end 94.929899 55.140101) (width 0.2) (layer "F.Cu") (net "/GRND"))
 (segment (start 69.73 85) (end 69.73 78.27) (width 0.2) (layer "F.Cu") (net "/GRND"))
 (segment (start 48.3 90.2075) (end 55.92 97.8275) (width 0.2) (layer "F.Cu") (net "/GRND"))
 (segment (start 74.5 73.5) (end 79.537056 73.5) (width 0.2) (layer "F.Cu") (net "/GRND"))
 (segment (start 79.165 90.24) (end 84.245 90.24) (width 0.2) (layer "F.Cu") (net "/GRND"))
 (segment (start 68.77 61.96) (end 88.11 61.96) (width 0.2) (layer "F.Cu") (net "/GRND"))
 (segment (start 68.81 42.5) (end 88 42.5) (width 0.2) (layer "F.Cu") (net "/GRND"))
 (segment (start 55.92 97.8275) (end 55.92 96.570265) (width 0.2) (layer "F.Cu") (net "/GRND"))
 (segment (start 92.05 58.02) (end 88.11 61.96) (width 0.2) (layer "F.Cu") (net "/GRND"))
 (segment (start 95.75 40.539899) (end 94.929899 41.36) (width 0.2) (layer "F.Cu") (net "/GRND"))
 (segment (start 79.165 90.24) (end 78.015 89.09) (width 0.2) (layer "F.Cu") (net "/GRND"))
 (segment (start 95.039899 60.82) (end 95.86 59.999899) (width 0.2) (layer "F.Cu") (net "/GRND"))
 (segment (start 78.015 89.09) (end 73.82 89.09) (width 0.2) (layer "F.Cu") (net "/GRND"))
 (segment (start 50.02 40.94) (end 51.46 39.5) (width 0.2) (layer "F.Cu") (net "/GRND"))
 (segment (start 95.039899 58.02) (end 92.05 58.02) (width 0.2) (layer "F.Cu") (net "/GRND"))
 (segment (start 67.77 60.96) (end 47.11 60.96) (width 0.2) (layer "F.Cu") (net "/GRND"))
 (segment (start 69.73 78.27) (end 70 78) (width 0.2) (layer "F.Cu") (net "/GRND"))
 (segment (start 95.75 39.380101) (end 95.75 40.539899) (width 0.2) (layer "F.Cu") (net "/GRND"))
 (segment (start 84.245 90.24) (end 91.865 97.86) (width 0.2) (layer "F.Cu") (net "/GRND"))
 (segment (start 76.19 90.19) (end 76.5 90.5) (width 0.2) (layer "F.Cu") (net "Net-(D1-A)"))
 (segment (start 72.27 85) (end 74.77 87.5) (width 0.2) (layer "F.Cu") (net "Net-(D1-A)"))
 (segment (start 74.77 87.5) (end 75 87.5) (width 0.2) (layer "F.Cu") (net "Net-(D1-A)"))
 (segment (start 74 90.19) (end 76.19 90.19) (width 0.2) (layer "F.Cu") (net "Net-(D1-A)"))
 (via (at 76.5 90.5) (size 0.6) (drill 0.3) (layers "F.Cu" "B.Cu") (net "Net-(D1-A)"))
 (via (at 74.77 87.5) (size 0.6) (drill 0.3) (layers "F.Cu" "B.Cu") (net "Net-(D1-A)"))
 (segment (start 69.5 90.19) (end 70.81 90.19) (width 0.2) (layer "F.Cu") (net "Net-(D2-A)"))
 (segment (start 70.81 90.19) (end 71.5 89.5) (width 0.2) (layer "F.Cu") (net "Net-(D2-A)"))
 (via (at 76 82.5) (size 0.6) (drill 0.3) (layers "F.Cu" "B.Cu") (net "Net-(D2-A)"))
 (via (at 71.5 89.5) (size 0.6) (drill 0.3) (layers "F.Cu" "B.Cu") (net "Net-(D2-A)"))
 (segment (start 70.75 58.75) (end 71 59) (width 0.2) (layer "F.Cu") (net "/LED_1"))
 (segment (start 60.18 51.1) (end 63.1 51.1) (width 0.2) (layer "F.Cu") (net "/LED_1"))
 (segment (start 63.1 51.1) (end 70.75 58.75) (width 0.2) (layer "F.Cu") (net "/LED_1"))
 (segment (start 74 97.81) (end 79.31 92.5) (width 0.2) (layer "F.Cu") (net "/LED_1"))
 (segment (start 59.08 52.2) (end 60.18 51.1) (width 0.2) (layer "F.Cu") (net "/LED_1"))
 (segment (start 79.31 92.5) (end 85 92.5) (width 0.2) (layer "F.Cu") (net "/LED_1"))
 (via (at 85 92.5) (size 0.6) (drill 0.3) (layers "F.Cu" "B.Cu") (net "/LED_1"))
 (via (at 70.75 58.75) (size 0.6) (drill 0.3) (layers "F.Cu" "B.Cu") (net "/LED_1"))
 (segment (start 64.75 58.75) (end 65 59) (width 0.2) (layer "F.Cu") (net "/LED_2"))
 (segment (start 69.5 97.81) (end 67.5 95.81) (width 0.2) (layer "F.Cu") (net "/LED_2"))
 (segment (start 61.62 52.2) (end 61.62 55.62) (width 0.2) (layer "F.Cu") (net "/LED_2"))
 (segment (start 61.62 55.62) (end 64.75 58.75) (width 0.2) (layer "F.Cu") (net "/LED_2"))
 (segment (start 67.5 95.81) (end 67.5 88.5) (width 0.2) (layer "F.Cu") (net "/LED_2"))
 (via (at 64.75 58.75) (size 0.6) (drill 0.3) (layers "F.Cu" "B.Cu") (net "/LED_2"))
 (via (at 67.5 88.5) (size 0.6) (drill 0.3) (layers "F.Cu" "B.Cu") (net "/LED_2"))
 (segment (start 94.35 47.107056) (end 80.637056 60.82) (width 0.2) (layer "F.Cu") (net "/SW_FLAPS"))
 (segment (start 61.799899 59.999899) (end 54 52.2) (width 0.2) (layer "F.Cu") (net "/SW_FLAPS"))
 (segment (start 80.637056 60.82) (end 74.540101 60.82) (width 0.2) (layer "F.Cu") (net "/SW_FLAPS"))
 (segment (start 74.540101 60.82) (end 73.72 59.999899) (width 0.2) (layer "F.Cu") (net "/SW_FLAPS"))
 (segment (start 73.72 59.999899) (end 61.799899 59.999899) (width 0.2) (layer "F.Cu") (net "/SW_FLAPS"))
 (segment (start 94.35 39.96) (end 94.35 47.107056) (width 0.2) (layer "F.Cu") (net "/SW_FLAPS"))
 (segment (start 75.12 59.42) (end 63.76 59.42) (width 0.2) (layer "F.Cu") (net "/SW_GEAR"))
 (segment (start 63.76 59.42) (end 56.54 52.2) (width 0.2) (layer "F.Cu") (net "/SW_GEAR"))
 (segment (start 62.04 39.92) (end 61.62 39.5) (width 0.2) (layer "F.Cu") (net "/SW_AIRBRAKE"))
 (segment (start 75.12 39.92) (end 62.04 39.92) (width 0.2) (layer "F.Cu") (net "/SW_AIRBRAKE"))
 (segment (start 53.46 58.42) (end 52.9 57.86) (width 0.2) (layer "F.Cu") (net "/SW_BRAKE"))
 (segment (start 52.9 45.68) (end 59.08 39.5) (width 0.2) (layer "F.Cu") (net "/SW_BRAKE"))
 (segment (start 52.9 57.86) (end 52.9 45.68) (width 0.2) (layer "F.Cu") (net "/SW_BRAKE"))
 (segment (start 50.946598 66.85) (end 45.71 61.613402) (width 0.2) (layer "F.Cu") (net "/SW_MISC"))
 (segment (start 47.689899 42.625736) (end 50.36 39.955635) (width 0.2) (layer "F.Cu") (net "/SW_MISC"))
 (segment (start 94.46 59.42) (end 92.629899 59.42) (width 0.2) (layer "F.Cu") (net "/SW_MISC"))
 (segment (start 92.629899 59.42) (end 88.689899 63.36) (width 0.2) (layer "F.Cu") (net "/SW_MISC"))
 (segment (start 87.530101 63.36) (end 86.71 62.539899) (width 0.2) (layer "F.Cu") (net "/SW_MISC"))
 (segment (start 45.71 61.613402) (end 45.71 60.380101) (width 0.2) (layer "F.Cu") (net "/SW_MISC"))
 (segment (start 88.689899 63.36) (end 87.530101 63.36) (width 0.2) (layer "F.Cu") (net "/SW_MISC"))
 (segment (start 47.689899 58.400202) (end 47.689899 42.625736) (width 0.2) (layer "F.Cu") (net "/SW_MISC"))
 (segment (start 82.399899 66.85) (end 50.946598 66.85) (width 0.2) (layer "F.Cu") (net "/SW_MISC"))
 (segment (start 51.004365 38.4) (end 55.44 38.4) (width 0.2) (layer "F.Cu") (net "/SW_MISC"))
 (segment (start 45.71 60.380101) (end 47.689899 58.400202) (width 0.2) (layer "F.Cu") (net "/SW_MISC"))
 (segment (start 50.36 39.955635) (end 50.36 39.044365) (width 0.2) (layer "F.Cu") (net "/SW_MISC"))
 (segment (start 86.71 62.539899) (end 82.399899 66.85) (width 0.2) (layer "F.Cu") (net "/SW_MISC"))
 (segment (start 50.36 39.044365) (end 51.004365 38.4) (width 0.2) (layer "F.Cu") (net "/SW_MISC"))
 (segment (start 55.44 38.4) (end 56.54 39.5) (width 0.2) (layer "F.Cu") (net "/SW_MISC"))
 (via (at 77 86.5) (size 0.6) (drill 0.3) (layers "F.Cu" "B.Cu") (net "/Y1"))
 (via (at 44.5 55) (size 0.6) (drill 0.3) (layers "F.Cu" "B.Cu") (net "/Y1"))
 (segment (start 48.92 57.58) (end 48.5 58) (width 0.2) (layer "F.Cu") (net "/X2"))
 (segment (start 48.92 52.2) (end 48.92 57.58) (width 0.2) (layer "F.Cu") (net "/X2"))
 (segment (start 53.38 97.8275) (end 53.38 96.88) (width 0.2) (layer "F.Cu") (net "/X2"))
 (segment (start 53.38 96.88) (end 48 91.5) (width 0.2) (layer "F.Cu") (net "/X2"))
 (via (at 48 91.5) (size 0.6) (drill 0.3) (layers "F.Cu" "B.Cu") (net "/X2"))
 (via (at 48.5 58) (size 0.6) (drill 0.3) (layers "F.Cu" "B.Cu") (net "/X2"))
 (segment (start 69.348529 86.5) (end 67.5 86.5) (width 0.2) (layer "F.Cu") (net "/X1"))
 (segment (start 84.777529 91.429) (end 73.683365 91.429) (width 0.2) (layer "F.Cu") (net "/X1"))
 (segment (start 89.325 97.86) (end 89.325 95.976471) (width 0.2) (layer "F.Cu") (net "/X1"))
 (segment (start 89.325 95.976471) (end 84.777529 91.429) (width 0.2) (layer "F.Cu") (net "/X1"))
 (segment (start 43.84 57.16) (end 43.5 57.5) (width 0.2) (layer "F.Cu") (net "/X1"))
 (segment (start 43.84 52.2) (end 43.84 57.16) (width 0.2) (layer "F.Cu") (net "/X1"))
 (segment (start 72.9 90.051471) (end 69.348529 86.5) (width 0.2) (layer "F.Cu") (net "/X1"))
 (segment (start 72.9 90.645635) (end 72.9 90.051471) (width 0.2) (layer "F.Cu") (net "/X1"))
 (segment (start 73.683365 91.429) (end 72.9 90.645635) (width 0.2) (layer "F.Cu") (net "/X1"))
 (via (at 67.5 86.5) (size 0.6) (drill 0.3) (layers "F.Cu" "B.Cu") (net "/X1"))
 (via (at 43.5 57.5) (size 0.6) (drill 0.3) (layers "F.Cu" "B.Cu") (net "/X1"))
 (segment (start 51.46 54.96) (end 51.5 55) (width 0.2) (layer "F.Cu") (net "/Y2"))
 (segment (start 44.317 81.597711) (end 44.317 58.183) (width 0.2) (layer "F.Cu") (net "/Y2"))
 (segment (start 44.5 86.3875) (end 44.5 81.780711) (width 0.2) (layer "F.Cu") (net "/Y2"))
 (segment (start 44.317 58.183) (end 46.5 56) (width 0.2) (layer "F.Cu") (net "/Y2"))
 (segment (start 51.46 52.2) (end 51.46 54.96) (width 0.2) (layer "F.Cu") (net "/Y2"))
 (segment (start 43.22 87.6675) (end 44.5 86.3875) (width 0.2) (layer "F.Cu") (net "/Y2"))
 (segment (start 44.5 81.780711) (end 44.317 81.597711) (width 0.2) (layer "F.Cu") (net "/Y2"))
 (via (at 46.5 56) (size 0.6) (drill 0.3) (layers "F.Cu" "B.Cu") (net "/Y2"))
 (via (at 51.5 55) (size 0.6) (drill 0.3) (layers "F.Cu" "B.Cu") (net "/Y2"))
 (segment (start 59.535635 38.4) (end 60.18 39.044365) (width 0.2) (layer "F.Cu") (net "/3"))
 (segment (start 60.18 46.664365) (end 55.1 51.744365) (width 0.2) (layer "F.Cu") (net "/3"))
 (segment (start 60.18 39.044365) (end 60.18 46.664365) (width 0.2) (layer "F.Cu") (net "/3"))
 (segment (start 71 81.848529) (end 71 81.5) (width 0.2) (layer "F.Cu") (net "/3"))
 (segment (start 57.98 39.044365) (end 58.624365 38.4) (width 0.2) (layer "F.Cu") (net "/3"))
 (segment (start 79.165 85.16) (end 78.725 85.6) (width 0.2) (layer "F.Cu") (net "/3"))
 (segment (start 58.624365 38.4) (end 59.535635 38.4) (width 0.2) (layer "F.Cu") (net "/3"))
 (segment (start 61.5 59) (end 62 59) (width 0.2) (layer "F.Cu") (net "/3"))
 (segment (start 55.1 52.6) (end 61.5 59) (width 0.2) (layer "F.Cu") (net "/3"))
 (segment (start 62 59) (end 62.5 59) (width 0.2) (layer "F.Cu") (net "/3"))
 (segment (start 78.725 85.6) (end 74.751471 85.6) (width 0.2) (layer "F.Cu") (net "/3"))
 (segment (start 50.84 97.8275) (end 50.84 96.34) (width 0.2) (layer "F.Cu") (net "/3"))
 (segment (start 80.66 85.16) (end 87.5 92) (width 0.2) (layer "F.Cu") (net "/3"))
 (segment (start 86.785 94.715) (end 87 94.5) (width 0.2) (layer "F.Cu") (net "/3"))
 (segment (start 74.751471 85.6) (end 71 81.848529) (width 0.2) (layer "F.Cu") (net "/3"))
 (segment (start 79.165 85.16) (end 80.66 85.16) (width 0.2) (layer "F.Cu") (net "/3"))
 (segment (start 43.22 85.1275) (end 43.22 82.28) (width 0.2) (layer "F.Cu") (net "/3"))
 (segment (start 43.22 82.28) (end 43.5 82) (width 0.2) (layer "F.Cu") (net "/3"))
 (segment (start 54 44.014314) (end 57.98 40.034314) (width 0.2) (layer "F.Cu") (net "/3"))
 (segment (start 55.1 51.744365) (end 55.1 52.6) (width 0.2) (layer "F.Cu") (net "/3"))
 (segment (start 50.84 96.34) (end 46 91.5) (width 0.2) (layer "F.Cu") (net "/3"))
 (segment (start 54 39.5) (end 54 44.014314) (width 0.2) (layer "F.Cu") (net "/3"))
 (segment (start 86.785 97.86) (end 86.785 94.715) (width 0.2) (layer "F.Cu") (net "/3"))
 (segment (start 57.98 40.034314) (end 57.98 39.044365) (width 0.2) (layer "F.Cu") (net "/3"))
 (via (at 43.5 82) (size 0.6) (drill 0.3) (layers "F.Cu" "B.Cu") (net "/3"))
 (via (at 46 91.5) (size 0.6) (drill 0.3) (layers "F.Cu" "B.Cu") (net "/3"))
 (via (at 71 81.5) (size 0.6) (drill 0.3) (layers "F.Cu" "B.Cu") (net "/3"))
 (via (at 87.5 92) (size 0.6) (drill 0.3) (layers "F.Cu" "B.Cu") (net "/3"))
 (via (at 87 94.5) (size 0.6) (drill 0.3) (layers "F.Cu" "B.Cu") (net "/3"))
 (via (at 62 59) (size 0.6) (drill 0.3) (layers "F.Cu" "B.Cu") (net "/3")))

